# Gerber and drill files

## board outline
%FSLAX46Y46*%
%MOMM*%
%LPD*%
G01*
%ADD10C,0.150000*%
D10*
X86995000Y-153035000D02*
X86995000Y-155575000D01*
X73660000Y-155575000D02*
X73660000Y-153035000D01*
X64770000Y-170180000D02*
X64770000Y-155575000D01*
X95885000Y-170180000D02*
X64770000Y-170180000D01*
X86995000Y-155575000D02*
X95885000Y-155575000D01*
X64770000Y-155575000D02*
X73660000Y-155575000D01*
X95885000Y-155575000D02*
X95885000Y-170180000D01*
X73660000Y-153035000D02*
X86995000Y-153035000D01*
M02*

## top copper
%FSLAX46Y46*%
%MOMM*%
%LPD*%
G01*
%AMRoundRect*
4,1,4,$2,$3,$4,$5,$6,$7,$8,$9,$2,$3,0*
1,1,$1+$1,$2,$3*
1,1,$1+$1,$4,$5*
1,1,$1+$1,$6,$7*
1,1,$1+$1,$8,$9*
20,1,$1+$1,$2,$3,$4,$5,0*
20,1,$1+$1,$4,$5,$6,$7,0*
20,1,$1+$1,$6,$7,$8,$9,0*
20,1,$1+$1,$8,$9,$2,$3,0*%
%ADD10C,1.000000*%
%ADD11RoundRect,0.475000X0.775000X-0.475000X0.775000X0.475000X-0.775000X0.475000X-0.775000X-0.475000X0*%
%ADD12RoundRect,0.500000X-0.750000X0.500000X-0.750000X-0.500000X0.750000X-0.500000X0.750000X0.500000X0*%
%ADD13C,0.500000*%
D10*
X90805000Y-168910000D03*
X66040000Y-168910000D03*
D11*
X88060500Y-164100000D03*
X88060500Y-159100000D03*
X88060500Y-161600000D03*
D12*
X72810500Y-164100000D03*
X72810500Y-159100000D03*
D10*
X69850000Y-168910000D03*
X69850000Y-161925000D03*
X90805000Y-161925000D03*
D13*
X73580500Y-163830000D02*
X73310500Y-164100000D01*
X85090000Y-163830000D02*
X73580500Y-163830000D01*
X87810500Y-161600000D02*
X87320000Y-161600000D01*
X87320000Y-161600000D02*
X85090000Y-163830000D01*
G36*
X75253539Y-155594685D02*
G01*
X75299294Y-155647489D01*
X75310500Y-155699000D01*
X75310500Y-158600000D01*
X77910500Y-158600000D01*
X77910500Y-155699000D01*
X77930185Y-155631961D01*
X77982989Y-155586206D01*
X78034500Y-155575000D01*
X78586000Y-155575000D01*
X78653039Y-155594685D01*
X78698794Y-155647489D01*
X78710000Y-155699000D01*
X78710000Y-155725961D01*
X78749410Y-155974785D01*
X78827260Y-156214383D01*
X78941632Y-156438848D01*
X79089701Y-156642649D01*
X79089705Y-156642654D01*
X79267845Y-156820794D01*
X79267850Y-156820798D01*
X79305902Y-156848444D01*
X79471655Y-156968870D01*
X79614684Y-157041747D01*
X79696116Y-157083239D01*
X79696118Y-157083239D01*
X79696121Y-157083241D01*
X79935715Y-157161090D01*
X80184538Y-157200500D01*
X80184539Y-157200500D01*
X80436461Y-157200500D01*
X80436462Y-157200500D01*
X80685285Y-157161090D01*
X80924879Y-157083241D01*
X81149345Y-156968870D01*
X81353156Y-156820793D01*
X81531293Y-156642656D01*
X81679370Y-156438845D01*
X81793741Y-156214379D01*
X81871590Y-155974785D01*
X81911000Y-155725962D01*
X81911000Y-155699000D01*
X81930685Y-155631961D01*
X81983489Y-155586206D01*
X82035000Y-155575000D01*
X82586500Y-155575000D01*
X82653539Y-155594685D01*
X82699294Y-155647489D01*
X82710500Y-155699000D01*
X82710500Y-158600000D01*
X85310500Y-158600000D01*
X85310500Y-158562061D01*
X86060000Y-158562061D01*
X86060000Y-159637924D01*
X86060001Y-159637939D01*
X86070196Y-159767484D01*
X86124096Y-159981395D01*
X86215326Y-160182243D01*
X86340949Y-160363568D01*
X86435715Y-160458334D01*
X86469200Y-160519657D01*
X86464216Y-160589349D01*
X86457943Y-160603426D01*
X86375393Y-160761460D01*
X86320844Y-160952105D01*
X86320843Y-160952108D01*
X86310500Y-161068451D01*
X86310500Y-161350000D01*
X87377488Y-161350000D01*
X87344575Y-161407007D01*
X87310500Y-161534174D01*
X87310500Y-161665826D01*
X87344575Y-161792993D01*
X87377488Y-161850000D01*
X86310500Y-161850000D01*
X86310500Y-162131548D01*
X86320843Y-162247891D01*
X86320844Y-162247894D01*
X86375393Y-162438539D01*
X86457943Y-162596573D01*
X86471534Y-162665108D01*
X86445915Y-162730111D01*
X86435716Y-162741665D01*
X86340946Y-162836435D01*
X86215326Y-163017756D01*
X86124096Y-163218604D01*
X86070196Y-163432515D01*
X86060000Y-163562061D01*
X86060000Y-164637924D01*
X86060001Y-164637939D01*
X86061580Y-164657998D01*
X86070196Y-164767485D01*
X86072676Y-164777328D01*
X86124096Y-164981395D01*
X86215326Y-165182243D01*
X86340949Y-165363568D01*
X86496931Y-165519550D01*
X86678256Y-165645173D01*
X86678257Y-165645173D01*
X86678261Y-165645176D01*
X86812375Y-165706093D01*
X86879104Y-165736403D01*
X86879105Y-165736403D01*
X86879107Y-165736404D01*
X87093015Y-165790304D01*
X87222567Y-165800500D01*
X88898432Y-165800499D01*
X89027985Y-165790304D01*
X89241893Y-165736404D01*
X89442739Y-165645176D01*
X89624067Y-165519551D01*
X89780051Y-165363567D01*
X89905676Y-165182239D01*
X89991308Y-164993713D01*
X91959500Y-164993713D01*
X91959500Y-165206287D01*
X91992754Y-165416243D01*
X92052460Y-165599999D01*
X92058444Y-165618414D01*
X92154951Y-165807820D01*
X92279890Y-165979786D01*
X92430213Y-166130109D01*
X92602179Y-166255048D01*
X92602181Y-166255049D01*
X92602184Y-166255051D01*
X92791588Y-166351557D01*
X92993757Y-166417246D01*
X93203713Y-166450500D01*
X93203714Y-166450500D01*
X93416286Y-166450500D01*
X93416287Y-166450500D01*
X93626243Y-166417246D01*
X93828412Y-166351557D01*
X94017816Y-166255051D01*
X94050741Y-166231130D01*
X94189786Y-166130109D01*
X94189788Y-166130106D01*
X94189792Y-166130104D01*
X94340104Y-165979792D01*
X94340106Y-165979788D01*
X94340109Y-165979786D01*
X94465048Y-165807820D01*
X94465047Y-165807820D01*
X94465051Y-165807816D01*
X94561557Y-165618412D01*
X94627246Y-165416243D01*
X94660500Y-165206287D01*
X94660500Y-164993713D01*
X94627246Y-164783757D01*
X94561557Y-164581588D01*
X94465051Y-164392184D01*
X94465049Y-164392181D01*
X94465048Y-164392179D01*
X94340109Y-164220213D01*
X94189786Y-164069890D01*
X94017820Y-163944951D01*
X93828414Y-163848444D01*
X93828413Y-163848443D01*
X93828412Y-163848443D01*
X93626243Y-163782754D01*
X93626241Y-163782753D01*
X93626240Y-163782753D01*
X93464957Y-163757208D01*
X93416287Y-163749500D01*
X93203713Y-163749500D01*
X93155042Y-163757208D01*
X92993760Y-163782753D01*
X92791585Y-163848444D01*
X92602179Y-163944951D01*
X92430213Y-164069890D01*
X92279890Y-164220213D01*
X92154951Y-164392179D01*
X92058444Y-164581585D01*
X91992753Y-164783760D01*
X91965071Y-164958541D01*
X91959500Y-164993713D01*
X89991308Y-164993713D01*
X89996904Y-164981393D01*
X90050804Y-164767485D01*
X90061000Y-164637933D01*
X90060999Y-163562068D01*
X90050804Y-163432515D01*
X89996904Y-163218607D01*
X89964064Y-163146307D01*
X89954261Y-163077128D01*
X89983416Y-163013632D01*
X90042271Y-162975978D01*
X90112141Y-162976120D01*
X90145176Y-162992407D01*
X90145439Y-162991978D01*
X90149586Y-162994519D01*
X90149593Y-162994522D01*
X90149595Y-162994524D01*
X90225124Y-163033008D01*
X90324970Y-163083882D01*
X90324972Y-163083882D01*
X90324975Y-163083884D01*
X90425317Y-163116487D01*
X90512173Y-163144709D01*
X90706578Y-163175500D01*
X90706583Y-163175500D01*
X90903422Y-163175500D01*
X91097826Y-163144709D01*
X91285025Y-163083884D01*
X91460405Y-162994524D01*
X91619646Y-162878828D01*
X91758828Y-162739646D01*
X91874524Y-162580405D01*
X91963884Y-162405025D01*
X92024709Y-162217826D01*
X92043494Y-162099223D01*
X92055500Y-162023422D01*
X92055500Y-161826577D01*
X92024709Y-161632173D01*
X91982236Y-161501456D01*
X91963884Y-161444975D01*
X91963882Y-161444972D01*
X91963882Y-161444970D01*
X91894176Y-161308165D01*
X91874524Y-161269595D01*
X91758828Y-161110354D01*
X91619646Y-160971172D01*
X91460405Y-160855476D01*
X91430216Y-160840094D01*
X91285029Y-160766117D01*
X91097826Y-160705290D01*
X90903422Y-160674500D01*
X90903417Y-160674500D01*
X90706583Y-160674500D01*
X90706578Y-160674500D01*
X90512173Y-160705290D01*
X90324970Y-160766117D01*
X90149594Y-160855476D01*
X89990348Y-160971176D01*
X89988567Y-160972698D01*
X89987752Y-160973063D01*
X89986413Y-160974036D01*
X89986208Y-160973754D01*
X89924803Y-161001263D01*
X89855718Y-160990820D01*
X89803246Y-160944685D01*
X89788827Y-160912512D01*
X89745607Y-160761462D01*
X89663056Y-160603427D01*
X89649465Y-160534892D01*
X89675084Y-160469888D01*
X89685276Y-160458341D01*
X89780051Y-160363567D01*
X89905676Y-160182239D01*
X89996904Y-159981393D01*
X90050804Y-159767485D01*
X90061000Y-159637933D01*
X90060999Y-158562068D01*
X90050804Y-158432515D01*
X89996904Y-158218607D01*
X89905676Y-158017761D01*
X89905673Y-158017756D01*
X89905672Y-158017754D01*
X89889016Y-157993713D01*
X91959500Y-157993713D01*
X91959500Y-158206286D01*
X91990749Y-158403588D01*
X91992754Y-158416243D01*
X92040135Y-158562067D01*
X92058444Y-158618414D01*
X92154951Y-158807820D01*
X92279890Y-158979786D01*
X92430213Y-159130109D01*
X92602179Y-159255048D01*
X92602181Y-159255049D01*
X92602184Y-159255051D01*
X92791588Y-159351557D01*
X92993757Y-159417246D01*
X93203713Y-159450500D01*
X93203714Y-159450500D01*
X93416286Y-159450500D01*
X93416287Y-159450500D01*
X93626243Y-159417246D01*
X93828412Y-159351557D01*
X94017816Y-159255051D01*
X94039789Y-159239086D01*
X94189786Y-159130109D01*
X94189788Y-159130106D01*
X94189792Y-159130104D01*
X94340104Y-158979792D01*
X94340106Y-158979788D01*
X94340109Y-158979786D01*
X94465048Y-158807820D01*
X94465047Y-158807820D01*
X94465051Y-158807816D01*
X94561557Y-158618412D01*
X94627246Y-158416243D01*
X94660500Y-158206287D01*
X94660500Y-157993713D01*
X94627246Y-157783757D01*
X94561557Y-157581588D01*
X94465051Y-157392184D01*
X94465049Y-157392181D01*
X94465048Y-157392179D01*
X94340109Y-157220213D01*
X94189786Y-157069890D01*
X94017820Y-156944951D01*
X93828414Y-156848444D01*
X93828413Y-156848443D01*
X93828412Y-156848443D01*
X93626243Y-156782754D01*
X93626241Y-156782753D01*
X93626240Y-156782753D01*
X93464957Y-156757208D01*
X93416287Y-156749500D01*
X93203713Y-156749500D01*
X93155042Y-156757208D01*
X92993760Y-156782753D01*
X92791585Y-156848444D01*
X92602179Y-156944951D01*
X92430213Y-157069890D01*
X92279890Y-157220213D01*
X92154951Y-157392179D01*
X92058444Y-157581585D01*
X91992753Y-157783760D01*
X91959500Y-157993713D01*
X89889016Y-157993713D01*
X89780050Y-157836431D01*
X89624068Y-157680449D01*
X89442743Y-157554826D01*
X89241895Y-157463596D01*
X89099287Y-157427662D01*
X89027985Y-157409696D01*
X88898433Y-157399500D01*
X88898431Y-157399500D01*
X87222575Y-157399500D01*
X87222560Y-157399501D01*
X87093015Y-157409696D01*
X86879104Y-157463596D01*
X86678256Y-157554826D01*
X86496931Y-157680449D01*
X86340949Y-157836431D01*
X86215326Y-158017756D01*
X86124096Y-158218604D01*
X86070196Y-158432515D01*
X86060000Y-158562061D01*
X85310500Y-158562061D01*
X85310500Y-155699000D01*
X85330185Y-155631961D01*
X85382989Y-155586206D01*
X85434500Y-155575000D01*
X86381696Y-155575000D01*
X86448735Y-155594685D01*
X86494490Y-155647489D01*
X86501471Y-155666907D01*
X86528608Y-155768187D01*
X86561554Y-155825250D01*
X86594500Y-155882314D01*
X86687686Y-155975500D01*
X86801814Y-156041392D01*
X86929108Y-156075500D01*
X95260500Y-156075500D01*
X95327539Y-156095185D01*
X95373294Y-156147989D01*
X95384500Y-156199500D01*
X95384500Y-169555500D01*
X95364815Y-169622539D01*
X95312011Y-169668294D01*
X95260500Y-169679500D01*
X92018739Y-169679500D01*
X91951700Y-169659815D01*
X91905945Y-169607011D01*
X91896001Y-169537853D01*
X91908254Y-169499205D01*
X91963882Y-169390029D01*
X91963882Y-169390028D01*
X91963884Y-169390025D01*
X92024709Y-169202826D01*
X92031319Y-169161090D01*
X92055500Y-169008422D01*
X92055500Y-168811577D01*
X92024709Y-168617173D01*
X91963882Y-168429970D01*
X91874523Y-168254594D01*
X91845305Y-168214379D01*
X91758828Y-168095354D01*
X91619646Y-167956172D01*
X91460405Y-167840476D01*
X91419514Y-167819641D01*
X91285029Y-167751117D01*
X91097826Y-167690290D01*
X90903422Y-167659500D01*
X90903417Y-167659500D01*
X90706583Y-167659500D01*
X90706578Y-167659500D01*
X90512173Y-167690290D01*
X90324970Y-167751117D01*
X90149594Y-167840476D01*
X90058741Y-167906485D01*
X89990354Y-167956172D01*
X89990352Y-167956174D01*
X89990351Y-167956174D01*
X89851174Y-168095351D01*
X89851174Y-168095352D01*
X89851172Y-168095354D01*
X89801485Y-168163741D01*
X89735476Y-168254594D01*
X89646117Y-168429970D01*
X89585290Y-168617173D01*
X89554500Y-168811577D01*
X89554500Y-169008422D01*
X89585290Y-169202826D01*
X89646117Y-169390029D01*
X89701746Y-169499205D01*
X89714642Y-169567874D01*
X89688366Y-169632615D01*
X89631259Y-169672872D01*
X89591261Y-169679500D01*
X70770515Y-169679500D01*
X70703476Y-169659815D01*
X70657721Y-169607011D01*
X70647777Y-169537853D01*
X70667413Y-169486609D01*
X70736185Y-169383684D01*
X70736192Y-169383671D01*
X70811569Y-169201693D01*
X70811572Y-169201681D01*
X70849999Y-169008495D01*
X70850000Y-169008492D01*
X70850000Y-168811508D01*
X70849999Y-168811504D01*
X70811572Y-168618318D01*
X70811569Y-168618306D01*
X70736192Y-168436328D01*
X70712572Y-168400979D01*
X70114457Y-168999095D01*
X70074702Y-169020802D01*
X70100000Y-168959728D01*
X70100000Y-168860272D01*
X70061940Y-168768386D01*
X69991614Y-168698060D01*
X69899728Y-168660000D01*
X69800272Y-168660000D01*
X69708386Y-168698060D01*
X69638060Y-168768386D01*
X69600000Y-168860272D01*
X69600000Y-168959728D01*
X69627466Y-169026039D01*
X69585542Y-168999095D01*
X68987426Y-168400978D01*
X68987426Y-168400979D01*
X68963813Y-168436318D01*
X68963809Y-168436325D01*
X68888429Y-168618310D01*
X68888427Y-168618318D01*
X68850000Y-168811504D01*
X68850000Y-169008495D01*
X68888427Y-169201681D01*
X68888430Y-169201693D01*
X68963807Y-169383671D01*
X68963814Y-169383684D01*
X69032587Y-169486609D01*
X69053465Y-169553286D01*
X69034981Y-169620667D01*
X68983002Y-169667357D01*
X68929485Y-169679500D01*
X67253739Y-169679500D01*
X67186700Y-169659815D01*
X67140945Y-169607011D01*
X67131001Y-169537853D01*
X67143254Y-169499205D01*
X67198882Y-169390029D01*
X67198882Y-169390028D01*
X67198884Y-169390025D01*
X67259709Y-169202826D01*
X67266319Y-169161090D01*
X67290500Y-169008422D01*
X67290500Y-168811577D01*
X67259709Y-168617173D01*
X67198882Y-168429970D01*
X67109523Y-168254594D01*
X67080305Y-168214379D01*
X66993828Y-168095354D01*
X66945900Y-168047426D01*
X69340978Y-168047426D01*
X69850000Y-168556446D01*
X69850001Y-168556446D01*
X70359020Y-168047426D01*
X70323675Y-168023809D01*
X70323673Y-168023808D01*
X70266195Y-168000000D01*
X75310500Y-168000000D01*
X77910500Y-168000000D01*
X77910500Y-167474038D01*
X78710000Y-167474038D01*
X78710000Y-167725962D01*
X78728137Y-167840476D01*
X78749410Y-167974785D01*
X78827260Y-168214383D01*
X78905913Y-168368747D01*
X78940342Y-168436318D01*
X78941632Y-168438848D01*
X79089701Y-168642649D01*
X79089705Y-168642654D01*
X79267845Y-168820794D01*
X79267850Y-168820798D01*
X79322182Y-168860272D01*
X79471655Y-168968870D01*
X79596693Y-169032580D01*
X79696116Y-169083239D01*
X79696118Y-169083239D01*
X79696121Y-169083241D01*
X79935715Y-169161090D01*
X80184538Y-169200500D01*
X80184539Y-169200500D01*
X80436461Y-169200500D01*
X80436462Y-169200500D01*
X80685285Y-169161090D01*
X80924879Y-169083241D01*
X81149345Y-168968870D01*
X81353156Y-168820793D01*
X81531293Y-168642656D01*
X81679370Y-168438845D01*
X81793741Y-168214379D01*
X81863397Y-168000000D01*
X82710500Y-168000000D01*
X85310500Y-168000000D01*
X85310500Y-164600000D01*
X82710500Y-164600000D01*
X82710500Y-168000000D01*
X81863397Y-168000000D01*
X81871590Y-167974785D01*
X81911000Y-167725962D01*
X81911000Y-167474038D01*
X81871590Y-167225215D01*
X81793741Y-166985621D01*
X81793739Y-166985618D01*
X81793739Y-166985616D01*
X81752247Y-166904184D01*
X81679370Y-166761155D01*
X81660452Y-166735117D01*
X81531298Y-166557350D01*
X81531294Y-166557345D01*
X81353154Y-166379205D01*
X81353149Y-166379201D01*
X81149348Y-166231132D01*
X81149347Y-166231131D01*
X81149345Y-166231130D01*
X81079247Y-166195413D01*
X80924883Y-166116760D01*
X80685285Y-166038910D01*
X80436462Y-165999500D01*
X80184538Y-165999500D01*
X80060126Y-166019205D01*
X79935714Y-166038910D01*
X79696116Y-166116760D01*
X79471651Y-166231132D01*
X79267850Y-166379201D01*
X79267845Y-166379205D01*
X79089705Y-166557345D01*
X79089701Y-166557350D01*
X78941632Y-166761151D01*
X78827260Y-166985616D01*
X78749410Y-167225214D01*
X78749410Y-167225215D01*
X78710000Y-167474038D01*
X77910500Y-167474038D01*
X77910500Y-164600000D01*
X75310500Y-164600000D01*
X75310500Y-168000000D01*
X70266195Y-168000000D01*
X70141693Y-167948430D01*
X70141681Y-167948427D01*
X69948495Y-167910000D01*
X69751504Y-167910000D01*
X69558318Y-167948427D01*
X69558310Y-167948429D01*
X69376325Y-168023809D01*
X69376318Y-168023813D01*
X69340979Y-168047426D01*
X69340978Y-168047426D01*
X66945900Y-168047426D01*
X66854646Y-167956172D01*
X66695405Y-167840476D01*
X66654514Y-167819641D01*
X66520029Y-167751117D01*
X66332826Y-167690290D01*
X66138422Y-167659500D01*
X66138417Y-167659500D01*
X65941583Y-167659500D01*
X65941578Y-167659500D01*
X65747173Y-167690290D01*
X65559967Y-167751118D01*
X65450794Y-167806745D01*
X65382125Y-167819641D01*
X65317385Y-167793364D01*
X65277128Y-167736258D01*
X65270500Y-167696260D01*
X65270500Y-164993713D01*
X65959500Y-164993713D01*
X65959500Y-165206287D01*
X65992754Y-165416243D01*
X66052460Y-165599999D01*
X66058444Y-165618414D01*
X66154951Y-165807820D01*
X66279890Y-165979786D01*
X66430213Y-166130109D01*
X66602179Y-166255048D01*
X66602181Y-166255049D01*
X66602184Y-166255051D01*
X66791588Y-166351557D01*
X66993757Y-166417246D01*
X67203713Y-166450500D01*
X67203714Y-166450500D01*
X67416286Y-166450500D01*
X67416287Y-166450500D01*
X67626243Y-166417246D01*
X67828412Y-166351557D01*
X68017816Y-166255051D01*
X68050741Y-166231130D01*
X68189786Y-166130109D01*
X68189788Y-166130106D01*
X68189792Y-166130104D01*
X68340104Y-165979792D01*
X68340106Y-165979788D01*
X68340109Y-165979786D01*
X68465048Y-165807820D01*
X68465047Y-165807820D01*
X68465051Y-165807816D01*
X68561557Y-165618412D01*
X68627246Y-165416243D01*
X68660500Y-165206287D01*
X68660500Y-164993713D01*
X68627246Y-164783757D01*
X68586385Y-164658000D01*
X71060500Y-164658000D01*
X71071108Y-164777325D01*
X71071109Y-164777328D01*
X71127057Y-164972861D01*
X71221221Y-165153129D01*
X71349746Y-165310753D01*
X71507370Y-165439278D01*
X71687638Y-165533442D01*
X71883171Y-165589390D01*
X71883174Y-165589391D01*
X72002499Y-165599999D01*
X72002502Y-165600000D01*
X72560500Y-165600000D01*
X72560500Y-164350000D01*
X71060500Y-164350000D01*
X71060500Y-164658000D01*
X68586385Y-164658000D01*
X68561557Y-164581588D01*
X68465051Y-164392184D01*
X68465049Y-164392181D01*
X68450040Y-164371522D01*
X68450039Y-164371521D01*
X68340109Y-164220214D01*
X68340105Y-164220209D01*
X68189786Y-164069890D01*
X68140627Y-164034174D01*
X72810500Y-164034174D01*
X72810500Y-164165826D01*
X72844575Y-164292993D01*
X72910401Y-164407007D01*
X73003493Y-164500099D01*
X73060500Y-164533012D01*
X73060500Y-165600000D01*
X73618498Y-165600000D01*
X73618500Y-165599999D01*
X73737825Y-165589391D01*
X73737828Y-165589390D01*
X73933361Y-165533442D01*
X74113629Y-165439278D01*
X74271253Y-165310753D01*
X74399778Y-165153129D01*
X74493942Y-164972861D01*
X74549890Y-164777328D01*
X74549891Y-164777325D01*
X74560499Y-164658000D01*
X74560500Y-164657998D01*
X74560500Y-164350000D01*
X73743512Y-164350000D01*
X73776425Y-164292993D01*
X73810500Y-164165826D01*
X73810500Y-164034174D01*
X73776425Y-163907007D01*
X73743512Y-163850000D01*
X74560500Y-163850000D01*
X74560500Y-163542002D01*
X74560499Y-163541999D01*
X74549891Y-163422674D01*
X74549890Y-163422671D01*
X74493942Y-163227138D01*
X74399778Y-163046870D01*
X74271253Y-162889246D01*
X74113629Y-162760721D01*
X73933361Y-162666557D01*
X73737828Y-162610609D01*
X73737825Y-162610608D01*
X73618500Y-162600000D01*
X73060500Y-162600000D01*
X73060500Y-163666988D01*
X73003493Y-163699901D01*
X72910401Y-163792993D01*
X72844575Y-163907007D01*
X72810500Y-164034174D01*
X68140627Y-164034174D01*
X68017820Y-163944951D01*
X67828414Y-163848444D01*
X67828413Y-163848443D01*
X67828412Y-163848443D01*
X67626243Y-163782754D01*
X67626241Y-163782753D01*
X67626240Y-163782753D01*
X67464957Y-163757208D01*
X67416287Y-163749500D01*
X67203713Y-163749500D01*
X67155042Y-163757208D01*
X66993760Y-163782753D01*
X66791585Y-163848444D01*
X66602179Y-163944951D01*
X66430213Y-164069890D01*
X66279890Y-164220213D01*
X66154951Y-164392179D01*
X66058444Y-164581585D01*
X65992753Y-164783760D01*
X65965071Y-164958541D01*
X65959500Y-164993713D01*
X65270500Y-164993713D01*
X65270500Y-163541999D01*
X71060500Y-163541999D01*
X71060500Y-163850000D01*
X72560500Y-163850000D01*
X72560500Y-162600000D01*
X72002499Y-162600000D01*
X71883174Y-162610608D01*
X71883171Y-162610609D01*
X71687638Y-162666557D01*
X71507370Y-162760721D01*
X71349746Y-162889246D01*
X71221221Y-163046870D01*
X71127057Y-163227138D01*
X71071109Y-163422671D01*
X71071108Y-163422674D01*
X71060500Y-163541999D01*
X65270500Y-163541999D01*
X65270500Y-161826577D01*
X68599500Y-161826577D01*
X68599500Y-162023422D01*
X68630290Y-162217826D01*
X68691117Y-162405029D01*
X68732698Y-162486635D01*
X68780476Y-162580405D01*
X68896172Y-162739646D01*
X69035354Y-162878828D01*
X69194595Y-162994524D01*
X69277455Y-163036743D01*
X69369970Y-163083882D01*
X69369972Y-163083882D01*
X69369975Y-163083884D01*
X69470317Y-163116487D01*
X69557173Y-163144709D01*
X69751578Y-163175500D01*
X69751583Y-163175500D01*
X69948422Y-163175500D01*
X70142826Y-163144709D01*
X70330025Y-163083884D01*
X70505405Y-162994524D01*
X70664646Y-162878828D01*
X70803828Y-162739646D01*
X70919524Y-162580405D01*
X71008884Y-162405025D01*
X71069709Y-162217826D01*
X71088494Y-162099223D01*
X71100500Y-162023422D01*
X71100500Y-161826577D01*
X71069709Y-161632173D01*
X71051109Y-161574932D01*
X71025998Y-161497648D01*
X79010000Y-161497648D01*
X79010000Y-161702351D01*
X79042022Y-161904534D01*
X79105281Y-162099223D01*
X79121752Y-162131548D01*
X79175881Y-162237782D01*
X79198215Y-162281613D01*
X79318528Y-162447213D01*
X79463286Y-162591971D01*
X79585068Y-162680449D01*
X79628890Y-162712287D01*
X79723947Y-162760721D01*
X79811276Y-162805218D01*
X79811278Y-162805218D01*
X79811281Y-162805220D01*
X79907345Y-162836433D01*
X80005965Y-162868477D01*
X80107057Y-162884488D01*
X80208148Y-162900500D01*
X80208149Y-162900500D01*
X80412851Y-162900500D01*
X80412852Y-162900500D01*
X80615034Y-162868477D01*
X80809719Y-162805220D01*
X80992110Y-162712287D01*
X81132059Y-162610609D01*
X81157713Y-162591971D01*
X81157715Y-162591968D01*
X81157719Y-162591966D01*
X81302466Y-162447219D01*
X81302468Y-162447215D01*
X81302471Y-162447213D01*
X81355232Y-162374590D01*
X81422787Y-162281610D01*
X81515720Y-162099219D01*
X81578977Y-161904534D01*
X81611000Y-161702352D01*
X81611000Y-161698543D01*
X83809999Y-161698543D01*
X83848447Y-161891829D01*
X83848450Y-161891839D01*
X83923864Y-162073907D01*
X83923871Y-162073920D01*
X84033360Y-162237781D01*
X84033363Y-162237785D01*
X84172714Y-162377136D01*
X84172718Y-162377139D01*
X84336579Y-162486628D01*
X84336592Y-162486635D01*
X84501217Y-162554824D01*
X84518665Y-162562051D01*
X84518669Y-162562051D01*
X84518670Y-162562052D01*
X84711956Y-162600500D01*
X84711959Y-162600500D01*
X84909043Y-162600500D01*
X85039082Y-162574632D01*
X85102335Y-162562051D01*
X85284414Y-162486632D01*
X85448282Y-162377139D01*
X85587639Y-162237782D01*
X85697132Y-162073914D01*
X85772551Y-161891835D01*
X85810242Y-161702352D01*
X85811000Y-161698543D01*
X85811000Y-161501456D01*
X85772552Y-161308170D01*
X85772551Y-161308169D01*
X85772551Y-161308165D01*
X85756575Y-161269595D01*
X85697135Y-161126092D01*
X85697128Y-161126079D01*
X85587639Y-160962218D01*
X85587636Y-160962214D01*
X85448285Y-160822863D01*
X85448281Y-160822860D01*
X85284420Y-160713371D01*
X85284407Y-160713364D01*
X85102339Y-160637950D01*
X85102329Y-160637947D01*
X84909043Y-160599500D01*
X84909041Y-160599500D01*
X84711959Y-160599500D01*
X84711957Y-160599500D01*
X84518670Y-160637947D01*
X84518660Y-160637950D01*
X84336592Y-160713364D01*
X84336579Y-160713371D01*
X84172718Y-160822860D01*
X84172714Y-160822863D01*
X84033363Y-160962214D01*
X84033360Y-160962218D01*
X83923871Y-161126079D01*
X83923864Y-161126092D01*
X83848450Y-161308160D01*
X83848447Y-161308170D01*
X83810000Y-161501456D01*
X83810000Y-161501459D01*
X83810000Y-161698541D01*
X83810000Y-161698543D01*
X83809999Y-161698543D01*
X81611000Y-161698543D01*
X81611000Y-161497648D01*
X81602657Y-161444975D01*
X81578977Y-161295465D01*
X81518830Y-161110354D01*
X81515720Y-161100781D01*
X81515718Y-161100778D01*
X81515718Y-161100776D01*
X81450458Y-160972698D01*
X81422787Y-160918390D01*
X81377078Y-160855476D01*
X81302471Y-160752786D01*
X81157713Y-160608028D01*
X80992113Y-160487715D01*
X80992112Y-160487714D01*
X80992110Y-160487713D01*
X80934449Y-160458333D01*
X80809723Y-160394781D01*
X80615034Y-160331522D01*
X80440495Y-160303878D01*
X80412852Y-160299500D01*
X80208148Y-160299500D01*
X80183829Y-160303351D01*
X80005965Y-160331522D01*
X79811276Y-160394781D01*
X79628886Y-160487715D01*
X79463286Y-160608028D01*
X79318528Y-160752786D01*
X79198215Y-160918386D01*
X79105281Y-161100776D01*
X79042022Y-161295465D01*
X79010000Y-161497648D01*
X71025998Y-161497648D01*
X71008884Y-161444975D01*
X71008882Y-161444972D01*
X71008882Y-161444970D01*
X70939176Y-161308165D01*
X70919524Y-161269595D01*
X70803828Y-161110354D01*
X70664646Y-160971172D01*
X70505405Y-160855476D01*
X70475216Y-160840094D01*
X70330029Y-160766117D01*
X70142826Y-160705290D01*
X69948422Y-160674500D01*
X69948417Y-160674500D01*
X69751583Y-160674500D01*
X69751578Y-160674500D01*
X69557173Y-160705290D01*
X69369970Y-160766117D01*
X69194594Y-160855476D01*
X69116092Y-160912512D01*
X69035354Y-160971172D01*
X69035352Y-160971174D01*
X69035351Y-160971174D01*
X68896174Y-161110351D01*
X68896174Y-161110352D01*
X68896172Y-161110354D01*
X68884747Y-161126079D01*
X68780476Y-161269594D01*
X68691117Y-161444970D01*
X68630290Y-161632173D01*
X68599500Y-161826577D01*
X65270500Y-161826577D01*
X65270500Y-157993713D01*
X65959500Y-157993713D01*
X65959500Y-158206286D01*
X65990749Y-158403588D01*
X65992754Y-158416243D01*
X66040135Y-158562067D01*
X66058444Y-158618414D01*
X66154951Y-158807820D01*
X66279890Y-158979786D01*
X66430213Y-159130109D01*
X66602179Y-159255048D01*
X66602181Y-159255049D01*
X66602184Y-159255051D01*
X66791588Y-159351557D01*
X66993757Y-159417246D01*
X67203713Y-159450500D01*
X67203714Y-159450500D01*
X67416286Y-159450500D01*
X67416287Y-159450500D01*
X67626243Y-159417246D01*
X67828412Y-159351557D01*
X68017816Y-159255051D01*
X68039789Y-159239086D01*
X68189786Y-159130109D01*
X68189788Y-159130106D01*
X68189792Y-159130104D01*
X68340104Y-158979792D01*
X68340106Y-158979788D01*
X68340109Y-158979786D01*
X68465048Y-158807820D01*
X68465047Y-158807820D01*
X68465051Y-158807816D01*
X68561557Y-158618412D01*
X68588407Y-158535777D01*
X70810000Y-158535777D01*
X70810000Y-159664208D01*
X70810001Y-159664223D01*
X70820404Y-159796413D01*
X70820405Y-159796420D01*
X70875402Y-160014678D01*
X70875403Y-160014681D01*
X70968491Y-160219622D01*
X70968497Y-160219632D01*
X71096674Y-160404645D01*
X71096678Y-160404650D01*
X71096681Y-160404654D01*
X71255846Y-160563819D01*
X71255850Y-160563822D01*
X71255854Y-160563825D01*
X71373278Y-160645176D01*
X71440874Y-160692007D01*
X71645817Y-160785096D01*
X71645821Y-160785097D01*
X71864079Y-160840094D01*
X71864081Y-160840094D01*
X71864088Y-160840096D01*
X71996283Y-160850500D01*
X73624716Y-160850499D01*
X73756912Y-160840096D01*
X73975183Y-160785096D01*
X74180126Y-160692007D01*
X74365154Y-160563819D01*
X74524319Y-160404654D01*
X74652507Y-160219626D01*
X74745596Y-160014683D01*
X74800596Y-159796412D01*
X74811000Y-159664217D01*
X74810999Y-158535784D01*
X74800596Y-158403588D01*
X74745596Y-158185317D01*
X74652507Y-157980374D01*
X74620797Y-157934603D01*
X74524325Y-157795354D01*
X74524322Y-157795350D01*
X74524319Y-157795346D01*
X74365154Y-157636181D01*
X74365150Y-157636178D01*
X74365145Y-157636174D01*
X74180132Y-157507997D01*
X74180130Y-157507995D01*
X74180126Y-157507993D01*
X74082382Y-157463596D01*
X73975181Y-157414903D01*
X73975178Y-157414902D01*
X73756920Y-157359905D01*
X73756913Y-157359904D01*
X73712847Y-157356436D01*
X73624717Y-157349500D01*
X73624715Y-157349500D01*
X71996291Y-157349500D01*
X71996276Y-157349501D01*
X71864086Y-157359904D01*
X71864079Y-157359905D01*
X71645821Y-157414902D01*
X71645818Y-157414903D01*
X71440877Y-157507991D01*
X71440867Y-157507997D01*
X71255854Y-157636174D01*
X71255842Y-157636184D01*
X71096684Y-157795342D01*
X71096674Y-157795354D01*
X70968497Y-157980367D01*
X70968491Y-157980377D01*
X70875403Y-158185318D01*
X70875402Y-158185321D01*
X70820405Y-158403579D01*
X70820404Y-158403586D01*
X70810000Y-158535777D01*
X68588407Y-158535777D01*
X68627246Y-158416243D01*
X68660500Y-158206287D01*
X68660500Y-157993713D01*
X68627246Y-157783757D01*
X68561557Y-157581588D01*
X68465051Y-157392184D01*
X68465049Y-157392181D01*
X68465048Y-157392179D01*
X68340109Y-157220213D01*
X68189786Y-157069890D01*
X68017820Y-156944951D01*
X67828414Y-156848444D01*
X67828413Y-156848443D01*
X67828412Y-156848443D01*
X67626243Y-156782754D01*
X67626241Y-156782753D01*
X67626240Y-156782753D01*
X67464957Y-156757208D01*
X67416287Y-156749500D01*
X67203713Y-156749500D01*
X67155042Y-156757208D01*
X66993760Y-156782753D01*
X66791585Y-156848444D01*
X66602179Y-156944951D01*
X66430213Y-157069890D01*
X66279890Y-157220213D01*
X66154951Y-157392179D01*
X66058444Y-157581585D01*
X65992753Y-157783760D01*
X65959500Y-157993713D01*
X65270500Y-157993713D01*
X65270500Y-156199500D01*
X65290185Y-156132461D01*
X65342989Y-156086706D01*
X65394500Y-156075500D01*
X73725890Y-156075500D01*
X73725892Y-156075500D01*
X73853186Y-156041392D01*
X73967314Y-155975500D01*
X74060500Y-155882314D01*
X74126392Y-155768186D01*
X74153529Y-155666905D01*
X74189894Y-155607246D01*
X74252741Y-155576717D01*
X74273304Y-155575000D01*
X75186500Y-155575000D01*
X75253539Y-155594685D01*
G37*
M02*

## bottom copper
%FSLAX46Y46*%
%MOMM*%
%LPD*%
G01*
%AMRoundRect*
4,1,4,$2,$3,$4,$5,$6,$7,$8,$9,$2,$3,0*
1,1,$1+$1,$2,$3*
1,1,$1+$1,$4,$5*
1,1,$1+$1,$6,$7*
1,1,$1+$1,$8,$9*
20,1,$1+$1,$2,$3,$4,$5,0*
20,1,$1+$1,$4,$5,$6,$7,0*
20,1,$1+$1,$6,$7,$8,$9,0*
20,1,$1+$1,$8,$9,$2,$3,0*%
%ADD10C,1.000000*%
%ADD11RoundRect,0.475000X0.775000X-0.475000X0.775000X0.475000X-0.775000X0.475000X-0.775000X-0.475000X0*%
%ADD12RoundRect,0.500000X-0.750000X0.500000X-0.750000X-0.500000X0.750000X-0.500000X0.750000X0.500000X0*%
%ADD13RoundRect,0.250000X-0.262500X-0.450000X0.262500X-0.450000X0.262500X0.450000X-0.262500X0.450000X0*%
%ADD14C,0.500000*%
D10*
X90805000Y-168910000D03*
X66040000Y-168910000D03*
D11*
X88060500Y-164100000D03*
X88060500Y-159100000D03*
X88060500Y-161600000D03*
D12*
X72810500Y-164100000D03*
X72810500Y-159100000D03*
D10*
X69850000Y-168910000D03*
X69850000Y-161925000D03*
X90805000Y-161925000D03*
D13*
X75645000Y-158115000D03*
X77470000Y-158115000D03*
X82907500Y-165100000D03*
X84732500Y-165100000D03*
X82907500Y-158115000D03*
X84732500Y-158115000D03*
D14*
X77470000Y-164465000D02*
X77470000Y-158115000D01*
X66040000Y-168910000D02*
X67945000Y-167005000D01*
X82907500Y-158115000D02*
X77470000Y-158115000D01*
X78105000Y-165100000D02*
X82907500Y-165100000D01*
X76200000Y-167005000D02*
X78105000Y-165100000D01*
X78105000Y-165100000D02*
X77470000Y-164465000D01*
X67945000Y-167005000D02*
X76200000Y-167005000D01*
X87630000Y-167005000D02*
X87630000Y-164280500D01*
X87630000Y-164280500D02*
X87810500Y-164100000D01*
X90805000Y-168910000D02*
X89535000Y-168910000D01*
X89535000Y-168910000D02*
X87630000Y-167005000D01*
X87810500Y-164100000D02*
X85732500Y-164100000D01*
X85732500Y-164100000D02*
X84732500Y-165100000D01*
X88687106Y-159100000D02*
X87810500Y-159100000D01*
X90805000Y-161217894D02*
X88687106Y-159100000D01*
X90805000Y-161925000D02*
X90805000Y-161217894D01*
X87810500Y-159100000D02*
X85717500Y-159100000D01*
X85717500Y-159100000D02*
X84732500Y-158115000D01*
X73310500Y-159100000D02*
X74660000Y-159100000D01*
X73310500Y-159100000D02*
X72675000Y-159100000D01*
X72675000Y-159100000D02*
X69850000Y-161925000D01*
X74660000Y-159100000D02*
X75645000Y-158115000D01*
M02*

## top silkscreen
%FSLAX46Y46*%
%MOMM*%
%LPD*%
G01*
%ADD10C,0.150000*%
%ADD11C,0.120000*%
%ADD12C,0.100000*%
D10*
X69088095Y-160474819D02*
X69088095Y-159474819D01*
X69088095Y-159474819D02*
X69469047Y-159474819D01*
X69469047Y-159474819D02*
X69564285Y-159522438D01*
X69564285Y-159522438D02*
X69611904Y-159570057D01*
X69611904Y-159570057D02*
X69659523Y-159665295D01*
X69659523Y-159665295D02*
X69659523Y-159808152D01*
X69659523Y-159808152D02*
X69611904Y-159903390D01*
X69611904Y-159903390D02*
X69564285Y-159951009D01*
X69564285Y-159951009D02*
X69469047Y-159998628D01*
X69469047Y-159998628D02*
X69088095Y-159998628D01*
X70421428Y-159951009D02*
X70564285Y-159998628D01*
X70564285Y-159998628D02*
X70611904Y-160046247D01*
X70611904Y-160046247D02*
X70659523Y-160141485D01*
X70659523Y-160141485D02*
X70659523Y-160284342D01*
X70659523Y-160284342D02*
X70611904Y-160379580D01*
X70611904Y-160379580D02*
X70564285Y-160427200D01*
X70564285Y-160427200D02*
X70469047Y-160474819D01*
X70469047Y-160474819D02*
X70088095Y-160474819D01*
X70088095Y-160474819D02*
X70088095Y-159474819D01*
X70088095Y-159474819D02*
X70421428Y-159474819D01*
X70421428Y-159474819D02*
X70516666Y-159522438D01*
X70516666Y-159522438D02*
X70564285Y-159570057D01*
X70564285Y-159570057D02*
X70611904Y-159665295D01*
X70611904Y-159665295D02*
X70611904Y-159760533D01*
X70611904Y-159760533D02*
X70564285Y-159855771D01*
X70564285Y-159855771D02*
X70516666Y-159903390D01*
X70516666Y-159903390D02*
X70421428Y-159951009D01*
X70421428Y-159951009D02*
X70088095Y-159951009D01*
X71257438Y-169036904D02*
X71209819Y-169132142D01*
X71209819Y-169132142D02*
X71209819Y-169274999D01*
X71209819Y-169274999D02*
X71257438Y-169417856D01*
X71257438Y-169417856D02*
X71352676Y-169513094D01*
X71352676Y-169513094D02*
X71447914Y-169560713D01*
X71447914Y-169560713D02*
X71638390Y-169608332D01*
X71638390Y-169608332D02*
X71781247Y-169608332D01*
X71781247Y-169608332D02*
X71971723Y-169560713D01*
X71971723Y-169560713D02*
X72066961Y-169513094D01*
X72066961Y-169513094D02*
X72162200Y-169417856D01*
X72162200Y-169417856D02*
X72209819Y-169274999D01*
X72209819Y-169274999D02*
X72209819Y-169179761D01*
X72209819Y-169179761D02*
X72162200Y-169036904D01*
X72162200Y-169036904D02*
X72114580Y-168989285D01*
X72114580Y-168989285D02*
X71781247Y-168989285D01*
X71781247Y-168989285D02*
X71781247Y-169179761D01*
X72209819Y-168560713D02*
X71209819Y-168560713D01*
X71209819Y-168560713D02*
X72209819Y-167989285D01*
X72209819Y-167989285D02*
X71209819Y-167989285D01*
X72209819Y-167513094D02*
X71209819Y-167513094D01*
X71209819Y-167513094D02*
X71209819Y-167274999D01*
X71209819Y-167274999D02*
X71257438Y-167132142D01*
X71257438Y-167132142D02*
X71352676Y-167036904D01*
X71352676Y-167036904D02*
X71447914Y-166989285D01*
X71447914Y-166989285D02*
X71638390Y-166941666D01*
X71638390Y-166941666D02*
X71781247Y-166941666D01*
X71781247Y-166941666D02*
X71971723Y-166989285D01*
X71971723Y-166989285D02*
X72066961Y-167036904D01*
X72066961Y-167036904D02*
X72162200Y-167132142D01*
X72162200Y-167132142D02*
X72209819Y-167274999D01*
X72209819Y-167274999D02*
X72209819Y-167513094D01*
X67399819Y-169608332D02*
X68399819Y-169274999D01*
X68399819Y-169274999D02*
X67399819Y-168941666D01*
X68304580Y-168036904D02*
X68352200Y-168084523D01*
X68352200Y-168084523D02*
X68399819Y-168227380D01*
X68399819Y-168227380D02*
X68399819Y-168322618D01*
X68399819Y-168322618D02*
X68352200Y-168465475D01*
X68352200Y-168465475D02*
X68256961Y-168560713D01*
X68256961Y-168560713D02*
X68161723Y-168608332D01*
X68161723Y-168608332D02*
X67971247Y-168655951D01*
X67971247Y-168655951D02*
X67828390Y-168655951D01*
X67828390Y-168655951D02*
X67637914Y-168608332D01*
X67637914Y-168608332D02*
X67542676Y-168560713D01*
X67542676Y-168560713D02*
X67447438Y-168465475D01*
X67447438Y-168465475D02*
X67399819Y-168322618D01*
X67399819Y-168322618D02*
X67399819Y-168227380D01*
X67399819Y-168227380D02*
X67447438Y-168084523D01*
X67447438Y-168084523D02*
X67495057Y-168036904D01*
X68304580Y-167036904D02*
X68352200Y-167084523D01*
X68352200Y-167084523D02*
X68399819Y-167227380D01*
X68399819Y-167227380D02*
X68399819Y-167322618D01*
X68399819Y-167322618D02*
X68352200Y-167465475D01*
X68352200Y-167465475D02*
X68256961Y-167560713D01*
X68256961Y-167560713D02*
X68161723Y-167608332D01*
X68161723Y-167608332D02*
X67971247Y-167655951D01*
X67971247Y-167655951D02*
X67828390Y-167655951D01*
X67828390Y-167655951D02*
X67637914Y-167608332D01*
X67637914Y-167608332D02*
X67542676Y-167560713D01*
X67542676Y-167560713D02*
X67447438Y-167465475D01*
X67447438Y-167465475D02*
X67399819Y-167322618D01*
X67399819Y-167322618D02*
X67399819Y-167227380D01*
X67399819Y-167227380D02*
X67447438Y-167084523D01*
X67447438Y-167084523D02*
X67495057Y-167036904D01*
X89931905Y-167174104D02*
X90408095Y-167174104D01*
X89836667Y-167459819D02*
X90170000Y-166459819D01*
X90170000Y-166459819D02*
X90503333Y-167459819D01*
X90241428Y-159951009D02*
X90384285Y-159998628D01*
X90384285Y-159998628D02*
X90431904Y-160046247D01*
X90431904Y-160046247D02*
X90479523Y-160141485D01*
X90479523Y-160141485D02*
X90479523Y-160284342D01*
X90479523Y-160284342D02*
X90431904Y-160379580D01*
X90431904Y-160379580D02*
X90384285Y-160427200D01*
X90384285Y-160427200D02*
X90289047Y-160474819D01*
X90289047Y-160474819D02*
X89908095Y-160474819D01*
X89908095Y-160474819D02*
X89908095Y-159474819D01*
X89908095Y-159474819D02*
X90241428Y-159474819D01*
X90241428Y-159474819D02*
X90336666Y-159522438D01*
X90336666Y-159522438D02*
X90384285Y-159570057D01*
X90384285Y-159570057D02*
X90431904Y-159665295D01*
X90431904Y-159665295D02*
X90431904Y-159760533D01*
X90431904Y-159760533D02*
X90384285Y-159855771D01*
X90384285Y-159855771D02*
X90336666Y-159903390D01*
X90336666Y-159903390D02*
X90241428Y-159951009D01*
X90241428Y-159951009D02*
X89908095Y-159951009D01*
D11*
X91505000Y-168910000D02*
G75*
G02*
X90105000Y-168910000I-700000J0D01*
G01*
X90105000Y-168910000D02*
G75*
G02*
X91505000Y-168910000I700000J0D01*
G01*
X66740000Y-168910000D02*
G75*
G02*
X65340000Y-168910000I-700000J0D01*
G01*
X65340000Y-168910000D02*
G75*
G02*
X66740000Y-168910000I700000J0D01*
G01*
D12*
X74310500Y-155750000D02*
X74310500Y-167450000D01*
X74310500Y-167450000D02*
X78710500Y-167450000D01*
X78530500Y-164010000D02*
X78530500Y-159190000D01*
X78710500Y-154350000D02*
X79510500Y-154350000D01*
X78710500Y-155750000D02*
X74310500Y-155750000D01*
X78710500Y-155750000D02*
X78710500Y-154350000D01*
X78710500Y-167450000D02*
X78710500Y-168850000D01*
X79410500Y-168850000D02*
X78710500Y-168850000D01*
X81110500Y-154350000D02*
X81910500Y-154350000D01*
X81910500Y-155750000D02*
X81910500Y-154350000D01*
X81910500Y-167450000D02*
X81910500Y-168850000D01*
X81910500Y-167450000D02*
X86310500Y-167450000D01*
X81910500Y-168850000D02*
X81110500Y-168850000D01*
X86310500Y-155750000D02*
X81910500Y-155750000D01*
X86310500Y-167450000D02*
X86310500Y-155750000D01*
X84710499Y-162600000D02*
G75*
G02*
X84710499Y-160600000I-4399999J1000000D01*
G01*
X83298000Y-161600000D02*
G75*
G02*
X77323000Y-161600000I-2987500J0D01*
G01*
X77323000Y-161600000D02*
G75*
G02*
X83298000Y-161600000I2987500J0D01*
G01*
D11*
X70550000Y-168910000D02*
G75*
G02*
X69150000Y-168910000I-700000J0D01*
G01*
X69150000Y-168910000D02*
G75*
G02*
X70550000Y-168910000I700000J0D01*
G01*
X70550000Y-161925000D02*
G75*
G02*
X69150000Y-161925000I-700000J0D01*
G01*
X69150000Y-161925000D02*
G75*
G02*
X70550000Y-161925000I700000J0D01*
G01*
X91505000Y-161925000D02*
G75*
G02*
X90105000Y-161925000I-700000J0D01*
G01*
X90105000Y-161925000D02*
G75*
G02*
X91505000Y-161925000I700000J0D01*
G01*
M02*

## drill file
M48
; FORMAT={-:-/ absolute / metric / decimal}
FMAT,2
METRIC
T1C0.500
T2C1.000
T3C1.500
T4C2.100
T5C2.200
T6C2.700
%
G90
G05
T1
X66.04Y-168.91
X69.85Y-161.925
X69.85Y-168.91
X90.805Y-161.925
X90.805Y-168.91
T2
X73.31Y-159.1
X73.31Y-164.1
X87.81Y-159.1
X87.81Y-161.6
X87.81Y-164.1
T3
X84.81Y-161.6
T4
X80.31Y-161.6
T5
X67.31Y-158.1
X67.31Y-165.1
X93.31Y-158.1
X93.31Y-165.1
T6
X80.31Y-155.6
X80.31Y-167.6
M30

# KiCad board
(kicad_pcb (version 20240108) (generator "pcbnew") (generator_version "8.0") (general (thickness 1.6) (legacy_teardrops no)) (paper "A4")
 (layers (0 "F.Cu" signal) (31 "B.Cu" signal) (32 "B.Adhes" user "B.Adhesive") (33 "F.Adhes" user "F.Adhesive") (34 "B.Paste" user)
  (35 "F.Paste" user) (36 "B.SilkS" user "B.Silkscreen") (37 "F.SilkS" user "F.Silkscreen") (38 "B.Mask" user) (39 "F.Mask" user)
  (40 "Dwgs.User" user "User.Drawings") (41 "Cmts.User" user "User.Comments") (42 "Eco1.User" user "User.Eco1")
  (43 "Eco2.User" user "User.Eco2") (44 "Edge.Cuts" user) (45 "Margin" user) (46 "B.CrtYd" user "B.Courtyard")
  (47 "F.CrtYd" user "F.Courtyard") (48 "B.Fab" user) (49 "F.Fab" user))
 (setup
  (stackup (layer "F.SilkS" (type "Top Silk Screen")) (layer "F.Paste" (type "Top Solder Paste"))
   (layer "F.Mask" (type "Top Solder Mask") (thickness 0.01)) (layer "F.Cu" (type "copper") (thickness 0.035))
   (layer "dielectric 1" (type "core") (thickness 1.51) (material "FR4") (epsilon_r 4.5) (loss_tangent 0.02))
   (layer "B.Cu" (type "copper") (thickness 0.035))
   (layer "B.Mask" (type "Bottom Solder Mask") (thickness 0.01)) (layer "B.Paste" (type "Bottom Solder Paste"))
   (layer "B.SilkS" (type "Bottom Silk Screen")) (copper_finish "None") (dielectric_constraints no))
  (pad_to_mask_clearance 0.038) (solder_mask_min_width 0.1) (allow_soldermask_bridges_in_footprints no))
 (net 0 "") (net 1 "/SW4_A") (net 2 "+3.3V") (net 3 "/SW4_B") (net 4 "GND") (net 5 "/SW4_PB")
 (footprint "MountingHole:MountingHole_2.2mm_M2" (layer "F.Cu") (at 67.31 165.1)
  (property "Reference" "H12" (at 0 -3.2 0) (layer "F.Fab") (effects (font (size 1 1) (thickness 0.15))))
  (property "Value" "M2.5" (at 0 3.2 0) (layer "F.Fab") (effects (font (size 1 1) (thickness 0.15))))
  (pad "" np_thru_hole circle (at 0 0) (size 2.2 2.2) (drill 2.2) (layers "*.Cu" "*.Mask")))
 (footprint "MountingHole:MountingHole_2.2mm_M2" (layer "F.Cu") (at 93.31 165.1)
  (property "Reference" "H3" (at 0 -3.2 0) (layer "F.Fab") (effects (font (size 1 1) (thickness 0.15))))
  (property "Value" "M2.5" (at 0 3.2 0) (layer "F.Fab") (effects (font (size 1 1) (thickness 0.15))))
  (pad "" np_thru_hole circle (at 0 0) (size 2.2 2.2) (drill 2.2) (layers "*.Cu" "*.Mask")))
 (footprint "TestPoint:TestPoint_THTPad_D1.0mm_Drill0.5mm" (layer "F.Cu") (at 90.805 168.91)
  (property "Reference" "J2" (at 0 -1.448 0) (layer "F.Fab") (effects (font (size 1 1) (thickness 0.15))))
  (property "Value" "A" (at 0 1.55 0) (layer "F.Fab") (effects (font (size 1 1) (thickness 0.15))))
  (fp_circle (center 0 0) (end 0 0.7) (stroke (width 0.12) (type solid)) (fill none) (layer "F.SilkS"))
  (pad "1" thru_hole circle (at 0 0) (size 1 1) (drill 0.5) (layers "*.Cu" "*.Mask") (remove_unused_layers no) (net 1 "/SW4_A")))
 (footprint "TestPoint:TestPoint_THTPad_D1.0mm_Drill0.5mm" (layer "F.Cu") (at 66.04 168.91)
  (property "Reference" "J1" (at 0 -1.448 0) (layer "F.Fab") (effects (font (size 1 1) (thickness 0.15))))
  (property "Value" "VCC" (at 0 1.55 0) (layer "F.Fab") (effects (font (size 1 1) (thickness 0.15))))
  (fp_circle (center 0 0) (end 0 0.7) (stroke (width 0.12) (type solid)) (fill none) (layer "F.SilkS"))
  (pad "1" thru_hole circle (at 0 0) (size 1 1) (drill 0.5) (layers "*.Cu" "*.Mask") (remove_unused_layers no) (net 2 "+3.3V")))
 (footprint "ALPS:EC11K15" (layer "F.Cu") (at 80.3105 161.6 90)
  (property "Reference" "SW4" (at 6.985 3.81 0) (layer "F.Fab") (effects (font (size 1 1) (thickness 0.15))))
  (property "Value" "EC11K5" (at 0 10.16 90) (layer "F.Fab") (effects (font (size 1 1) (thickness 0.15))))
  (fp_line (start 5.85 -6) (end -5.85 -6) (stroke (width 0.1) (type solid)) (layer "F.SilkS"))
  (fp_line (start -5.85 -6) (end -5.85 -1.6) (stroke (width 0.1) (type solid)) (layer "F.SilkS"))
  (fp_line (start -2.41 -1.78) (end 2.41 -1.78) (stroke (width 0.1) (type solid)) (layer "F.SilkS"))
  (fp_line (start 7.25 -1.6) (end 7.25 -0.8) (stroke (width 0.1) (type solid)) (layer "F.SilkS"))
  (fp_line (start 5.85 -1.6) (end 5.85 -6) (stroke (width 0.1) (type solid)) (layer "F.SilkS"))
  (fp_line (start 5.85 -1.6) (end 7.25 -1.6) (stroke (width 0.1) (type solid)) (layer "F.SilkS"))
  (fp_line (start -5.85 -1.6) (end -7.25 -1.6) (stroke (width 0.1) (type solid)) (layer "F.SilkS"))
  (fp_line (start -7.25 -0.9) (end -7.25 -1.6) (stroke (width 0.1) (type solid)) (layer "F.SilkS"))
  (fp_line (start 7.25 0.8) (end 7.25 1.6) (stroke (width 0.1) (type solid)) (layer "F.SilkS"))
  (fp_line (start 5.85 1.6) (end 7.25 1.6) (stroke (width 0.1) (type solid)) (layer "F.SilkS"))
  (fp_line (start -5.85 1.6) (end -7.25 1.6) (stroke (width 0.1) (type solid)) (layer "F.SilkS"))
  (fp_line (start -5.85 1.6) (end -5.85 6) (stroke (width 0.1) (type solid)) (layer "F.SilkS"))
  (fp_line (start -7.25 1.6) (end -7.25 0.8) (stroke (width 0.1) (type solid)) (layer "F.SilkS"))
  (fp_line (start 5.85 6) (end 5.85 1.6) (stroke (width 0.1) (type solid)) (layer "F.SilkS"))
  (fp_line (start -5.85 6) (end 5.85 6) (stroke (width 0.1) (type solid)) (layer "F.SilkS"))
  (fp_arc (start -1 4.399999) (mid 0 -4.512205) (end 1 4.399999) (stroke (width 0.1) (type solid)) (layer "F.SilkS"))
  (fp_circle (center 0 0) (end 2.9875 0) (stroke (width 0.1) (type solid)) (fill none) (layer "F.SilkS"))
  (pad "" np_thru_hole circle (at -6 0 90) (size 2.7 2.7) (drill 2.7) (layers "*.Cu" "*.Mask"))
  (pad "" np_thru_hole circle (at 0 0 90) (size 2.1 2.1) (drill 2.1) (layers "*.Cu" "*.Mask"))
  (pad "" np_thru_hole circle (at 0 4.5 90) (size 1.5 1.5) (drill 1.5) (layers "*.Cu" "*.Mask"))
  (pad "" np_thru_hole circle (at 6 0 90) (size 2.7 2.7) (drill 2.7) (layers "*.Cu" "*.Mask"))
  (pad "A" thru_hole roundrect (at -2.5 7.5 90) (size 1.9 2.5) (drill 1 (offset 0 0.25)) (layers "*.Cu" "*.Mask") (remove_unused_layers no)
   (roundrect_rratio 0.25) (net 1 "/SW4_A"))
  (pad "B" thru_hole roundrect (at 2.5 7.5 90) (size 1.9 2.5) (drill 1 (offset 0 0.25)) (layers "*.Cu" "*.Mask") (remove_unused_layers no)
   (roundrect_rratio 0.25) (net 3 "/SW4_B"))
  (pad "C" thru_hole roundrect (at 0 7.5 90) (size 1.9 2.5) (drill 1 (offset 0 0.25)) (layers "*.Cu" "*.Mask") (remove_unused_layers no)
   (roundrect_rratio 0.25) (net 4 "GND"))
  (pad "S1" thru_hole roundrect (at -2.5 -7 270) (size 2 2.5) (drill 1 (offset 0 0.5)) (layers "*.Cu" "*.Mask") (remove_unused_layers no)
   (roundrect_rratio 0.25) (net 4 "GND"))
  (pad "S2" thru_hole roundrect (at 2.5 -7 270) (size 2 2.5) (drill 1 (offset 0 0.5)) (layers "*.Cu" "*.Mask") (remove_unused_layers no)
   (roundrect_rratio 0.25) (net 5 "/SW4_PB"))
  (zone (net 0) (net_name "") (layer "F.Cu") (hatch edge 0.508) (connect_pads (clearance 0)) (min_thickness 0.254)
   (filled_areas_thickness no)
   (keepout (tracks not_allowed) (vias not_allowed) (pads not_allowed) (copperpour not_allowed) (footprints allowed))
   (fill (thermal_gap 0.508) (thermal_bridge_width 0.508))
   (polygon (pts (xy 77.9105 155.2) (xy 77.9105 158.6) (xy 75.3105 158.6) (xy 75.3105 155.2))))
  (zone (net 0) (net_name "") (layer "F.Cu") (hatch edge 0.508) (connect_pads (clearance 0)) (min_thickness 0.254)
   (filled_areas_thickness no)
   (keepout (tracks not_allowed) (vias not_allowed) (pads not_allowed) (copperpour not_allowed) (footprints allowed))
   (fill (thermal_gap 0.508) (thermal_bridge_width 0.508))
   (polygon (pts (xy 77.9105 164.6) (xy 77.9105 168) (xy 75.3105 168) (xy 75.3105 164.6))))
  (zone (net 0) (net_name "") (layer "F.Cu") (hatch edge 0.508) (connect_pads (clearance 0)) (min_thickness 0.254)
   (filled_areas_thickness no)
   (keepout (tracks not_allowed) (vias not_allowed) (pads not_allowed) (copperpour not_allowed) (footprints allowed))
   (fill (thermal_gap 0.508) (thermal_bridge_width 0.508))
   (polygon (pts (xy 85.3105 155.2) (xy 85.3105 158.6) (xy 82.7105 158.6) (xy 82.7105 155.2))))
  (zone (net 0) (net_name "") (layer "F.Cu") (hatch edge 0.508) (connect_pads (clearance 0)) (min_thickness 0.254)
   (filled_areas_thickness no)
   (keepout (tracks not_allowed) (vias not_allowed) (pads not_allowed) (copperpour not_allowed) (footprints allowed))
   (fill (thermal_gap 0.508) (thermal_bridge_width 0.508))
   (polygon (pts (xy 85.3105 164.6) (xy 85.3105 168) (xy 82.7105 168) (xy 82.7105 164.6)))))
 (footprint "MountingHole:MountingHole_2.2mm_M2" (layer "F.Cu") (at 67.31 158.1)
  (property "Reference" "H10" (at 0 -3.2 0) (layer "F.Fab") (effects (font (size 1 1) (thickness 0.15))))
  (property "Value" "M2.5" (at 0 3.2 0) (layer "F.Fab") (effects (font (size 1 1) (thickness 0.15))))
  (pad "" np_thru_hole circle (at 0 0) (size 2.2 2.2) (drill 2.2) (layers "*.Cu" "*.Mask")))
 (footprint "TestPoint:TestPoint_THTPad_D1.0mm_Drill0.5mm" (layer "F.Cu") (at 69.85 168.91)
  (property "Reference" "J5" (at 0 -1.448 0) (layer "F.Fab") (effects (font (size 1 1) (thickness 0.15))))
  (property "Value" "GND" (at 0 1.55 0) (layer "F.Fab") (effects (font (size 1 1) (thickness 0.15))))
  (fp_circle (center 0 0) (end 0 0.7) (stroke (width 0.12) (type solid)) (fill none) (layer "F.SilkS"))
  (pad "1" thru_hole circle (at 0 0) (size 1 1) (drill 0.5) (layers "*.Cu" "*.Mask") (remove_unused_layers no) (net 4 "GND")))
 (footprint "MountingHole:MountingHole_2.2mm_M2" (layer "F.Cu") (at 93.31 158.1)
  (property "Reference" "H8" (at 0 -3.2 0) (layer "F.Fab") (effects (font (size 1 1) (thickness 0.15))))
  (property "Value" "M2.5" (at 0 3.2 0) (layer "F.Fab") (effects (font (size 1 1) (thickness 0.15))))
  (pad "" np_thru_hole circle (at 0 0) (size 2.2 2.2) (drill 2.2) (layers "*.Cu" "*.Mask")))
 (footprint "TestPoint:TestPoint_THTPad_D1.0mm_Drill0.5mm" (layer "F.Cu") (at 69.85 161.925)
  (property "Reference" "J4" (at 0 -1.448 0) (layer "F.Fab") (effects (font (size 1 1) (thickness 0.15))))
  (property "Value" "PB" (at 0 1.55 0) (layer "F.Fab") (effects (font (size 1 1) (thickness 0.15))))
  (fp_circle (center 0 0) (end 0 0.7) (stroke (width 0.12) (type solid)) (fill none) (layer "F.SilkS"))
  (pad "1" thru_hole circle (at 0 0) (size 1 1) (drill 0.5) (layers "*.Cu" "*.Mask") (remove_unused_layers no) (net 5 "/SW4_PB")))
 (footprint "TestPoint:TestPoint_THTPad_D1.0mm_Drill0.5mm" (layer "F.Cu") (at 90.805 161.925)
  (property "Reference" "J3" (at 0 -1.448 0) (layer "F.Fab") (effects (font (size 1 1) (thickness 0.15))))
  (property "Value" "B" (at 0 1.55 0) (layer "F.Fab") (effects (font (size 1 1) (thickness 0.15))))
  (fp_circle (center 0 0) (end 0 0.7) (stroke (width 0.12) (type solid)) (fill none) (layer "F.SilkS"))
  (pad "1" thru_hole circle (at 0 0) (size 1 1) (drill 0.5) (layers "*.Cu" "*.Mask") (remove_unused_layers no) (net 3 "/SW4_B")))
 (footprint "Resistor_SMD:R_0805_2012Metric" (layer "B.Cu") (at 76.5575 158.115)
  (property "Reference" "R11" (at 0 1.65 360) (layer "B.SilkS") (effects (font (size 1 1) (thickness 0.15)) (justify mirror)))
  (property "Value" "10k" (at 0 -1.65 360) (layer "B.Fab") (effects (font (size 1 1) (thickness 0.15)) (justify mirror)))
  (pad "1" smd roundrect (at -0.9125 0) (size 1.025 1.4) (layers "B.Cu" "B.Paste" "B.Mask") (roundrect_rratio 0.243902) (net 5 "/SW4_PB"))
  (pad "2" smd roundrect (at 0.9125 0) (size 1.025 1.4) (layers "B.Cu" "B.Paste" "B.Mask") (roundrect_rratio 0.243902) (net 2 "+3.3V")))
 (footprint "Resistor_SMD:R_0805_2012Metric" (layer "B.Cu") (at 83.82 165.1)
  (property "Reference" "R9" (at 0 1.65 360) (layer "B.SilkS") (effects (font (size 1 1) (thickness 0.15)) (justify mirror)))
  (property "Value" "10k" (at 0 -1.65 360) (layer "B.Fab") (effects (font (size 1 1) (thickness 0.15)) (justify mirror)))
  (pad "1" smd roundrect (at -0.9125 0) (size 1.025 1.4) (layers "B.Cu" "B.Paste" "B.Mask") (roundrect_rratio 0.243902) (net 2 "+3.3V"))
  (pad "2" smd roundrect (at 0.9125 0) (size 1.025 1.4) (layers "B.Cu" "B.Paste" "B.Mask") (roundrect_rratio 0.243902) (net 1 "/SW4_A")))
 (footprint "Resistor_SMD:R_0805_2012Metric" (layer "B.Cu") (at 83.82 158.115)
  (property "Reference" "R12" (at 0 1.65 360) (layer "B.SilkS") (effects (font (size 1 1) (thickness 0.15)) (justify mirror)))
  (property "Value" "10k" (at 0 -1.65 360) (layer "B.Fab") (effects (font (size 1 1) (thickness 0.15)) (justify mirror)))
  (pad "1" smd roundrect (at -0.9125 0) (size 1.025 1.4) (layers "B.Cu" "B.Paste" "B.Mask") (roundrect_rratio 0.243902) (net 2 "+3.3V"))
  (pad "2" smd roundrect (at 0.9125 0) (size 1.025 1.4) (layers "B.Cu" "B.Paste" "B.Mask") (roundrect_rratio 0.243902) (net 3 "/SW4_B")))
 (gr_line (start 86.995 153.035) (end 86.995 155.575) (stroke (width 0.15) (type default)) (layer "Edge.Cuts"))
 (gr_line (start 73.66 155.575) (end 73.66 153.035) (stroke (width 0.15) (type default)) (layer "Edge.Cuts"))
 (gr_line (start 64.77 170.18) (end 64.77 155.575) (stroke (width 0.15) (type default)) (layer "Edge.Cuts"))
 (gr_line (start 95.885 170.18) (end 64.77 170.18) (stroke (width 0.15) (type default)) (layer "Edge.Cuts"))
 (gr_line (start 86.995 155.575) (end 95.885 155.575) (stroke (width 0.15) (type default)) (layer "Edge.Cuts"))
 (gr_line (start 64.77 155.575) (end 73.66 155.575) (stroke (width 0.15) (type default)) (layer "Edge.Cuts"))
 (gr_line (start 95.885 155.575) (end 95.885 170.18) (stroke (width 0.15) (type default)) (layer "Edge.Cuts"))
 (gr_line (start 73.66 153.035) (end 86.995 153.035) (stroke (width 0.15) (type default)) (layer "Edge.Cuts"))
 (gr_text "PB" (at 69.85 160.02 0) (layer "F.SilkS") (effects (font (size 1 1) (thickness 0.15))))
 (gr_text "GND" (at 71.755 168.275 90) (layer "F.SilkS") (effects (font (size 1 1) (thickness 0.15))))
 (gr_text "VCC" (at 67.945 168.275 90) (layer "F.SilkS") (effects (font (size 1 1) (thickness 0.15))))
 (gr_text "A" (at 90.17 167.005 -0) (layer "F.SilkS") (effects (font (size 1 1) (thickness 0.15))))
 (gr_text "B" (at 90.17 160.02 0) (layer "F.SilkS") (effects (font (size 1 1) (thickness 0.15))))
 (segment (start 73.5805 163.83) (end 73.3105 164.1) (width 0.5) (layer "F.Cu") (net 4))
 (segment (start 85.09 163.83) (end 73.5805 163.83) (width 0.5) (layer "F.Cu") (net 4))
 (segment (start 87.8105 161.6) (end 87.32 161.6) (width 0.5) (layer "F.Cu") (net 4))
 (segment (start 87.32 161.6) (end 85.09 163.83) (width 0.5) (layer "F.Cu") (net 4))
 (segment (start 77.47 164.465) (end 77.47 158.115) (width 0.5) (layer "B.Cu") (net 2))
 (segment (start 66.04 168.91) (end 67.945 167.005) (width 0.5) (layer "B.Cu") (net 2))
 (segment (start 82.9075 158.115) (end 77.47 158.115) (width 0.5) (layer "B.Cu") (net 2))
 (segment (start 78.105 165.1) (end 82.9075 165.1) (width 0.5) (layer "B.Cu") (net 2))
 (segment (start 76.2 167.005) (end 78.105 165.1) (width 0.5) (layer "B.Cu") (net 2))
 (segment (start 78.105 165.1) (end 77.47 164.465) (width 0.5) (layer "B.Cu") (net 2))
 (segment (start 67.945 167.005) (end 76.2 167.005) (width 0.5) (layer "B.Cu") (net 2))
 (segment (start 87.63 167.005) (end 87.63 164.2805) (width 0.5) (layer "B.Cu") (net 1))
 (segment (start 87.63 164.2805) (end 87.8105 164.1) (width 0.5) (layer "B.Cu") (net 1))
 (segment (start 90.805 168.91) (end 89.535 168.91) (width 0.5) (layer "B.Cu") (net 1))
 (segment (start 89.535 168.91) (end 87.63 167.005) (width 0.5) (layer "B.Cu") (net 1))
 (segment (start 87.8105 164.1) (end 85.7325 164.1) (width 0.5) (layer "B.Cu") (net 1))
 (segment (start 85.7325 164.1) (end 84.7325 165.1) (width 0.5) (layer "B.Cu") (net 1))
 (segment (start 88.687106 159.1) (end 87.8105 159.1) (width 0.5) (layer "B.Cu") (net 3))
 (segment (start 90.805 161.217894) (end 88.687106 159.1) (width 0.5) (layer "B.Cu") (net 3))
 (segment (start 90.805 161.925) (end 90.805 161.217894) (width 0.5) (layer "B.Cu") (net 3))
 (segment (start 87.8105 159.1) (end 85.7175 159.1) (width 0.5) (layer "B.Cu") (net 3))
 (segment (start 85.7175 159.1) (end 84.7325 158.115) (width 0.5) (layer "B.Cu") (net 3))
 (segment (start 73.3105 159.1) (end 74.66 159.1) (width 0.5) (layer "B.Cu") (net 5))
 (segment (start 73.3105 159.1) (end 72.675 159.1) (width 0.5) (layer "B.Cu") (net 5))
 (segment (start 72.675 159.1) (end 69.85 161.925) (width 0.5) (layer "B.Cu") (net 5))
 (segment (start 74.66 159.1) (end 75.645 158.115) (width 0.5) (layer "B.Cu") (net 5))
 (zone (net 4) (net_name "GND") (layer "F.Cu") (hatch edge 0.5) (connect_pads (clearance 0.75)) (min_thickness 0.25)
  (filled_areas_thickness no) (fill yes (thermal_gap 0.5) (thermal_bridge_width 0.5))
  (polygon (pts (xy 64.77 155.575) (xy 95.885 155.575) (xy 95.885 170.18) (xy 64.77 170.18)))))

